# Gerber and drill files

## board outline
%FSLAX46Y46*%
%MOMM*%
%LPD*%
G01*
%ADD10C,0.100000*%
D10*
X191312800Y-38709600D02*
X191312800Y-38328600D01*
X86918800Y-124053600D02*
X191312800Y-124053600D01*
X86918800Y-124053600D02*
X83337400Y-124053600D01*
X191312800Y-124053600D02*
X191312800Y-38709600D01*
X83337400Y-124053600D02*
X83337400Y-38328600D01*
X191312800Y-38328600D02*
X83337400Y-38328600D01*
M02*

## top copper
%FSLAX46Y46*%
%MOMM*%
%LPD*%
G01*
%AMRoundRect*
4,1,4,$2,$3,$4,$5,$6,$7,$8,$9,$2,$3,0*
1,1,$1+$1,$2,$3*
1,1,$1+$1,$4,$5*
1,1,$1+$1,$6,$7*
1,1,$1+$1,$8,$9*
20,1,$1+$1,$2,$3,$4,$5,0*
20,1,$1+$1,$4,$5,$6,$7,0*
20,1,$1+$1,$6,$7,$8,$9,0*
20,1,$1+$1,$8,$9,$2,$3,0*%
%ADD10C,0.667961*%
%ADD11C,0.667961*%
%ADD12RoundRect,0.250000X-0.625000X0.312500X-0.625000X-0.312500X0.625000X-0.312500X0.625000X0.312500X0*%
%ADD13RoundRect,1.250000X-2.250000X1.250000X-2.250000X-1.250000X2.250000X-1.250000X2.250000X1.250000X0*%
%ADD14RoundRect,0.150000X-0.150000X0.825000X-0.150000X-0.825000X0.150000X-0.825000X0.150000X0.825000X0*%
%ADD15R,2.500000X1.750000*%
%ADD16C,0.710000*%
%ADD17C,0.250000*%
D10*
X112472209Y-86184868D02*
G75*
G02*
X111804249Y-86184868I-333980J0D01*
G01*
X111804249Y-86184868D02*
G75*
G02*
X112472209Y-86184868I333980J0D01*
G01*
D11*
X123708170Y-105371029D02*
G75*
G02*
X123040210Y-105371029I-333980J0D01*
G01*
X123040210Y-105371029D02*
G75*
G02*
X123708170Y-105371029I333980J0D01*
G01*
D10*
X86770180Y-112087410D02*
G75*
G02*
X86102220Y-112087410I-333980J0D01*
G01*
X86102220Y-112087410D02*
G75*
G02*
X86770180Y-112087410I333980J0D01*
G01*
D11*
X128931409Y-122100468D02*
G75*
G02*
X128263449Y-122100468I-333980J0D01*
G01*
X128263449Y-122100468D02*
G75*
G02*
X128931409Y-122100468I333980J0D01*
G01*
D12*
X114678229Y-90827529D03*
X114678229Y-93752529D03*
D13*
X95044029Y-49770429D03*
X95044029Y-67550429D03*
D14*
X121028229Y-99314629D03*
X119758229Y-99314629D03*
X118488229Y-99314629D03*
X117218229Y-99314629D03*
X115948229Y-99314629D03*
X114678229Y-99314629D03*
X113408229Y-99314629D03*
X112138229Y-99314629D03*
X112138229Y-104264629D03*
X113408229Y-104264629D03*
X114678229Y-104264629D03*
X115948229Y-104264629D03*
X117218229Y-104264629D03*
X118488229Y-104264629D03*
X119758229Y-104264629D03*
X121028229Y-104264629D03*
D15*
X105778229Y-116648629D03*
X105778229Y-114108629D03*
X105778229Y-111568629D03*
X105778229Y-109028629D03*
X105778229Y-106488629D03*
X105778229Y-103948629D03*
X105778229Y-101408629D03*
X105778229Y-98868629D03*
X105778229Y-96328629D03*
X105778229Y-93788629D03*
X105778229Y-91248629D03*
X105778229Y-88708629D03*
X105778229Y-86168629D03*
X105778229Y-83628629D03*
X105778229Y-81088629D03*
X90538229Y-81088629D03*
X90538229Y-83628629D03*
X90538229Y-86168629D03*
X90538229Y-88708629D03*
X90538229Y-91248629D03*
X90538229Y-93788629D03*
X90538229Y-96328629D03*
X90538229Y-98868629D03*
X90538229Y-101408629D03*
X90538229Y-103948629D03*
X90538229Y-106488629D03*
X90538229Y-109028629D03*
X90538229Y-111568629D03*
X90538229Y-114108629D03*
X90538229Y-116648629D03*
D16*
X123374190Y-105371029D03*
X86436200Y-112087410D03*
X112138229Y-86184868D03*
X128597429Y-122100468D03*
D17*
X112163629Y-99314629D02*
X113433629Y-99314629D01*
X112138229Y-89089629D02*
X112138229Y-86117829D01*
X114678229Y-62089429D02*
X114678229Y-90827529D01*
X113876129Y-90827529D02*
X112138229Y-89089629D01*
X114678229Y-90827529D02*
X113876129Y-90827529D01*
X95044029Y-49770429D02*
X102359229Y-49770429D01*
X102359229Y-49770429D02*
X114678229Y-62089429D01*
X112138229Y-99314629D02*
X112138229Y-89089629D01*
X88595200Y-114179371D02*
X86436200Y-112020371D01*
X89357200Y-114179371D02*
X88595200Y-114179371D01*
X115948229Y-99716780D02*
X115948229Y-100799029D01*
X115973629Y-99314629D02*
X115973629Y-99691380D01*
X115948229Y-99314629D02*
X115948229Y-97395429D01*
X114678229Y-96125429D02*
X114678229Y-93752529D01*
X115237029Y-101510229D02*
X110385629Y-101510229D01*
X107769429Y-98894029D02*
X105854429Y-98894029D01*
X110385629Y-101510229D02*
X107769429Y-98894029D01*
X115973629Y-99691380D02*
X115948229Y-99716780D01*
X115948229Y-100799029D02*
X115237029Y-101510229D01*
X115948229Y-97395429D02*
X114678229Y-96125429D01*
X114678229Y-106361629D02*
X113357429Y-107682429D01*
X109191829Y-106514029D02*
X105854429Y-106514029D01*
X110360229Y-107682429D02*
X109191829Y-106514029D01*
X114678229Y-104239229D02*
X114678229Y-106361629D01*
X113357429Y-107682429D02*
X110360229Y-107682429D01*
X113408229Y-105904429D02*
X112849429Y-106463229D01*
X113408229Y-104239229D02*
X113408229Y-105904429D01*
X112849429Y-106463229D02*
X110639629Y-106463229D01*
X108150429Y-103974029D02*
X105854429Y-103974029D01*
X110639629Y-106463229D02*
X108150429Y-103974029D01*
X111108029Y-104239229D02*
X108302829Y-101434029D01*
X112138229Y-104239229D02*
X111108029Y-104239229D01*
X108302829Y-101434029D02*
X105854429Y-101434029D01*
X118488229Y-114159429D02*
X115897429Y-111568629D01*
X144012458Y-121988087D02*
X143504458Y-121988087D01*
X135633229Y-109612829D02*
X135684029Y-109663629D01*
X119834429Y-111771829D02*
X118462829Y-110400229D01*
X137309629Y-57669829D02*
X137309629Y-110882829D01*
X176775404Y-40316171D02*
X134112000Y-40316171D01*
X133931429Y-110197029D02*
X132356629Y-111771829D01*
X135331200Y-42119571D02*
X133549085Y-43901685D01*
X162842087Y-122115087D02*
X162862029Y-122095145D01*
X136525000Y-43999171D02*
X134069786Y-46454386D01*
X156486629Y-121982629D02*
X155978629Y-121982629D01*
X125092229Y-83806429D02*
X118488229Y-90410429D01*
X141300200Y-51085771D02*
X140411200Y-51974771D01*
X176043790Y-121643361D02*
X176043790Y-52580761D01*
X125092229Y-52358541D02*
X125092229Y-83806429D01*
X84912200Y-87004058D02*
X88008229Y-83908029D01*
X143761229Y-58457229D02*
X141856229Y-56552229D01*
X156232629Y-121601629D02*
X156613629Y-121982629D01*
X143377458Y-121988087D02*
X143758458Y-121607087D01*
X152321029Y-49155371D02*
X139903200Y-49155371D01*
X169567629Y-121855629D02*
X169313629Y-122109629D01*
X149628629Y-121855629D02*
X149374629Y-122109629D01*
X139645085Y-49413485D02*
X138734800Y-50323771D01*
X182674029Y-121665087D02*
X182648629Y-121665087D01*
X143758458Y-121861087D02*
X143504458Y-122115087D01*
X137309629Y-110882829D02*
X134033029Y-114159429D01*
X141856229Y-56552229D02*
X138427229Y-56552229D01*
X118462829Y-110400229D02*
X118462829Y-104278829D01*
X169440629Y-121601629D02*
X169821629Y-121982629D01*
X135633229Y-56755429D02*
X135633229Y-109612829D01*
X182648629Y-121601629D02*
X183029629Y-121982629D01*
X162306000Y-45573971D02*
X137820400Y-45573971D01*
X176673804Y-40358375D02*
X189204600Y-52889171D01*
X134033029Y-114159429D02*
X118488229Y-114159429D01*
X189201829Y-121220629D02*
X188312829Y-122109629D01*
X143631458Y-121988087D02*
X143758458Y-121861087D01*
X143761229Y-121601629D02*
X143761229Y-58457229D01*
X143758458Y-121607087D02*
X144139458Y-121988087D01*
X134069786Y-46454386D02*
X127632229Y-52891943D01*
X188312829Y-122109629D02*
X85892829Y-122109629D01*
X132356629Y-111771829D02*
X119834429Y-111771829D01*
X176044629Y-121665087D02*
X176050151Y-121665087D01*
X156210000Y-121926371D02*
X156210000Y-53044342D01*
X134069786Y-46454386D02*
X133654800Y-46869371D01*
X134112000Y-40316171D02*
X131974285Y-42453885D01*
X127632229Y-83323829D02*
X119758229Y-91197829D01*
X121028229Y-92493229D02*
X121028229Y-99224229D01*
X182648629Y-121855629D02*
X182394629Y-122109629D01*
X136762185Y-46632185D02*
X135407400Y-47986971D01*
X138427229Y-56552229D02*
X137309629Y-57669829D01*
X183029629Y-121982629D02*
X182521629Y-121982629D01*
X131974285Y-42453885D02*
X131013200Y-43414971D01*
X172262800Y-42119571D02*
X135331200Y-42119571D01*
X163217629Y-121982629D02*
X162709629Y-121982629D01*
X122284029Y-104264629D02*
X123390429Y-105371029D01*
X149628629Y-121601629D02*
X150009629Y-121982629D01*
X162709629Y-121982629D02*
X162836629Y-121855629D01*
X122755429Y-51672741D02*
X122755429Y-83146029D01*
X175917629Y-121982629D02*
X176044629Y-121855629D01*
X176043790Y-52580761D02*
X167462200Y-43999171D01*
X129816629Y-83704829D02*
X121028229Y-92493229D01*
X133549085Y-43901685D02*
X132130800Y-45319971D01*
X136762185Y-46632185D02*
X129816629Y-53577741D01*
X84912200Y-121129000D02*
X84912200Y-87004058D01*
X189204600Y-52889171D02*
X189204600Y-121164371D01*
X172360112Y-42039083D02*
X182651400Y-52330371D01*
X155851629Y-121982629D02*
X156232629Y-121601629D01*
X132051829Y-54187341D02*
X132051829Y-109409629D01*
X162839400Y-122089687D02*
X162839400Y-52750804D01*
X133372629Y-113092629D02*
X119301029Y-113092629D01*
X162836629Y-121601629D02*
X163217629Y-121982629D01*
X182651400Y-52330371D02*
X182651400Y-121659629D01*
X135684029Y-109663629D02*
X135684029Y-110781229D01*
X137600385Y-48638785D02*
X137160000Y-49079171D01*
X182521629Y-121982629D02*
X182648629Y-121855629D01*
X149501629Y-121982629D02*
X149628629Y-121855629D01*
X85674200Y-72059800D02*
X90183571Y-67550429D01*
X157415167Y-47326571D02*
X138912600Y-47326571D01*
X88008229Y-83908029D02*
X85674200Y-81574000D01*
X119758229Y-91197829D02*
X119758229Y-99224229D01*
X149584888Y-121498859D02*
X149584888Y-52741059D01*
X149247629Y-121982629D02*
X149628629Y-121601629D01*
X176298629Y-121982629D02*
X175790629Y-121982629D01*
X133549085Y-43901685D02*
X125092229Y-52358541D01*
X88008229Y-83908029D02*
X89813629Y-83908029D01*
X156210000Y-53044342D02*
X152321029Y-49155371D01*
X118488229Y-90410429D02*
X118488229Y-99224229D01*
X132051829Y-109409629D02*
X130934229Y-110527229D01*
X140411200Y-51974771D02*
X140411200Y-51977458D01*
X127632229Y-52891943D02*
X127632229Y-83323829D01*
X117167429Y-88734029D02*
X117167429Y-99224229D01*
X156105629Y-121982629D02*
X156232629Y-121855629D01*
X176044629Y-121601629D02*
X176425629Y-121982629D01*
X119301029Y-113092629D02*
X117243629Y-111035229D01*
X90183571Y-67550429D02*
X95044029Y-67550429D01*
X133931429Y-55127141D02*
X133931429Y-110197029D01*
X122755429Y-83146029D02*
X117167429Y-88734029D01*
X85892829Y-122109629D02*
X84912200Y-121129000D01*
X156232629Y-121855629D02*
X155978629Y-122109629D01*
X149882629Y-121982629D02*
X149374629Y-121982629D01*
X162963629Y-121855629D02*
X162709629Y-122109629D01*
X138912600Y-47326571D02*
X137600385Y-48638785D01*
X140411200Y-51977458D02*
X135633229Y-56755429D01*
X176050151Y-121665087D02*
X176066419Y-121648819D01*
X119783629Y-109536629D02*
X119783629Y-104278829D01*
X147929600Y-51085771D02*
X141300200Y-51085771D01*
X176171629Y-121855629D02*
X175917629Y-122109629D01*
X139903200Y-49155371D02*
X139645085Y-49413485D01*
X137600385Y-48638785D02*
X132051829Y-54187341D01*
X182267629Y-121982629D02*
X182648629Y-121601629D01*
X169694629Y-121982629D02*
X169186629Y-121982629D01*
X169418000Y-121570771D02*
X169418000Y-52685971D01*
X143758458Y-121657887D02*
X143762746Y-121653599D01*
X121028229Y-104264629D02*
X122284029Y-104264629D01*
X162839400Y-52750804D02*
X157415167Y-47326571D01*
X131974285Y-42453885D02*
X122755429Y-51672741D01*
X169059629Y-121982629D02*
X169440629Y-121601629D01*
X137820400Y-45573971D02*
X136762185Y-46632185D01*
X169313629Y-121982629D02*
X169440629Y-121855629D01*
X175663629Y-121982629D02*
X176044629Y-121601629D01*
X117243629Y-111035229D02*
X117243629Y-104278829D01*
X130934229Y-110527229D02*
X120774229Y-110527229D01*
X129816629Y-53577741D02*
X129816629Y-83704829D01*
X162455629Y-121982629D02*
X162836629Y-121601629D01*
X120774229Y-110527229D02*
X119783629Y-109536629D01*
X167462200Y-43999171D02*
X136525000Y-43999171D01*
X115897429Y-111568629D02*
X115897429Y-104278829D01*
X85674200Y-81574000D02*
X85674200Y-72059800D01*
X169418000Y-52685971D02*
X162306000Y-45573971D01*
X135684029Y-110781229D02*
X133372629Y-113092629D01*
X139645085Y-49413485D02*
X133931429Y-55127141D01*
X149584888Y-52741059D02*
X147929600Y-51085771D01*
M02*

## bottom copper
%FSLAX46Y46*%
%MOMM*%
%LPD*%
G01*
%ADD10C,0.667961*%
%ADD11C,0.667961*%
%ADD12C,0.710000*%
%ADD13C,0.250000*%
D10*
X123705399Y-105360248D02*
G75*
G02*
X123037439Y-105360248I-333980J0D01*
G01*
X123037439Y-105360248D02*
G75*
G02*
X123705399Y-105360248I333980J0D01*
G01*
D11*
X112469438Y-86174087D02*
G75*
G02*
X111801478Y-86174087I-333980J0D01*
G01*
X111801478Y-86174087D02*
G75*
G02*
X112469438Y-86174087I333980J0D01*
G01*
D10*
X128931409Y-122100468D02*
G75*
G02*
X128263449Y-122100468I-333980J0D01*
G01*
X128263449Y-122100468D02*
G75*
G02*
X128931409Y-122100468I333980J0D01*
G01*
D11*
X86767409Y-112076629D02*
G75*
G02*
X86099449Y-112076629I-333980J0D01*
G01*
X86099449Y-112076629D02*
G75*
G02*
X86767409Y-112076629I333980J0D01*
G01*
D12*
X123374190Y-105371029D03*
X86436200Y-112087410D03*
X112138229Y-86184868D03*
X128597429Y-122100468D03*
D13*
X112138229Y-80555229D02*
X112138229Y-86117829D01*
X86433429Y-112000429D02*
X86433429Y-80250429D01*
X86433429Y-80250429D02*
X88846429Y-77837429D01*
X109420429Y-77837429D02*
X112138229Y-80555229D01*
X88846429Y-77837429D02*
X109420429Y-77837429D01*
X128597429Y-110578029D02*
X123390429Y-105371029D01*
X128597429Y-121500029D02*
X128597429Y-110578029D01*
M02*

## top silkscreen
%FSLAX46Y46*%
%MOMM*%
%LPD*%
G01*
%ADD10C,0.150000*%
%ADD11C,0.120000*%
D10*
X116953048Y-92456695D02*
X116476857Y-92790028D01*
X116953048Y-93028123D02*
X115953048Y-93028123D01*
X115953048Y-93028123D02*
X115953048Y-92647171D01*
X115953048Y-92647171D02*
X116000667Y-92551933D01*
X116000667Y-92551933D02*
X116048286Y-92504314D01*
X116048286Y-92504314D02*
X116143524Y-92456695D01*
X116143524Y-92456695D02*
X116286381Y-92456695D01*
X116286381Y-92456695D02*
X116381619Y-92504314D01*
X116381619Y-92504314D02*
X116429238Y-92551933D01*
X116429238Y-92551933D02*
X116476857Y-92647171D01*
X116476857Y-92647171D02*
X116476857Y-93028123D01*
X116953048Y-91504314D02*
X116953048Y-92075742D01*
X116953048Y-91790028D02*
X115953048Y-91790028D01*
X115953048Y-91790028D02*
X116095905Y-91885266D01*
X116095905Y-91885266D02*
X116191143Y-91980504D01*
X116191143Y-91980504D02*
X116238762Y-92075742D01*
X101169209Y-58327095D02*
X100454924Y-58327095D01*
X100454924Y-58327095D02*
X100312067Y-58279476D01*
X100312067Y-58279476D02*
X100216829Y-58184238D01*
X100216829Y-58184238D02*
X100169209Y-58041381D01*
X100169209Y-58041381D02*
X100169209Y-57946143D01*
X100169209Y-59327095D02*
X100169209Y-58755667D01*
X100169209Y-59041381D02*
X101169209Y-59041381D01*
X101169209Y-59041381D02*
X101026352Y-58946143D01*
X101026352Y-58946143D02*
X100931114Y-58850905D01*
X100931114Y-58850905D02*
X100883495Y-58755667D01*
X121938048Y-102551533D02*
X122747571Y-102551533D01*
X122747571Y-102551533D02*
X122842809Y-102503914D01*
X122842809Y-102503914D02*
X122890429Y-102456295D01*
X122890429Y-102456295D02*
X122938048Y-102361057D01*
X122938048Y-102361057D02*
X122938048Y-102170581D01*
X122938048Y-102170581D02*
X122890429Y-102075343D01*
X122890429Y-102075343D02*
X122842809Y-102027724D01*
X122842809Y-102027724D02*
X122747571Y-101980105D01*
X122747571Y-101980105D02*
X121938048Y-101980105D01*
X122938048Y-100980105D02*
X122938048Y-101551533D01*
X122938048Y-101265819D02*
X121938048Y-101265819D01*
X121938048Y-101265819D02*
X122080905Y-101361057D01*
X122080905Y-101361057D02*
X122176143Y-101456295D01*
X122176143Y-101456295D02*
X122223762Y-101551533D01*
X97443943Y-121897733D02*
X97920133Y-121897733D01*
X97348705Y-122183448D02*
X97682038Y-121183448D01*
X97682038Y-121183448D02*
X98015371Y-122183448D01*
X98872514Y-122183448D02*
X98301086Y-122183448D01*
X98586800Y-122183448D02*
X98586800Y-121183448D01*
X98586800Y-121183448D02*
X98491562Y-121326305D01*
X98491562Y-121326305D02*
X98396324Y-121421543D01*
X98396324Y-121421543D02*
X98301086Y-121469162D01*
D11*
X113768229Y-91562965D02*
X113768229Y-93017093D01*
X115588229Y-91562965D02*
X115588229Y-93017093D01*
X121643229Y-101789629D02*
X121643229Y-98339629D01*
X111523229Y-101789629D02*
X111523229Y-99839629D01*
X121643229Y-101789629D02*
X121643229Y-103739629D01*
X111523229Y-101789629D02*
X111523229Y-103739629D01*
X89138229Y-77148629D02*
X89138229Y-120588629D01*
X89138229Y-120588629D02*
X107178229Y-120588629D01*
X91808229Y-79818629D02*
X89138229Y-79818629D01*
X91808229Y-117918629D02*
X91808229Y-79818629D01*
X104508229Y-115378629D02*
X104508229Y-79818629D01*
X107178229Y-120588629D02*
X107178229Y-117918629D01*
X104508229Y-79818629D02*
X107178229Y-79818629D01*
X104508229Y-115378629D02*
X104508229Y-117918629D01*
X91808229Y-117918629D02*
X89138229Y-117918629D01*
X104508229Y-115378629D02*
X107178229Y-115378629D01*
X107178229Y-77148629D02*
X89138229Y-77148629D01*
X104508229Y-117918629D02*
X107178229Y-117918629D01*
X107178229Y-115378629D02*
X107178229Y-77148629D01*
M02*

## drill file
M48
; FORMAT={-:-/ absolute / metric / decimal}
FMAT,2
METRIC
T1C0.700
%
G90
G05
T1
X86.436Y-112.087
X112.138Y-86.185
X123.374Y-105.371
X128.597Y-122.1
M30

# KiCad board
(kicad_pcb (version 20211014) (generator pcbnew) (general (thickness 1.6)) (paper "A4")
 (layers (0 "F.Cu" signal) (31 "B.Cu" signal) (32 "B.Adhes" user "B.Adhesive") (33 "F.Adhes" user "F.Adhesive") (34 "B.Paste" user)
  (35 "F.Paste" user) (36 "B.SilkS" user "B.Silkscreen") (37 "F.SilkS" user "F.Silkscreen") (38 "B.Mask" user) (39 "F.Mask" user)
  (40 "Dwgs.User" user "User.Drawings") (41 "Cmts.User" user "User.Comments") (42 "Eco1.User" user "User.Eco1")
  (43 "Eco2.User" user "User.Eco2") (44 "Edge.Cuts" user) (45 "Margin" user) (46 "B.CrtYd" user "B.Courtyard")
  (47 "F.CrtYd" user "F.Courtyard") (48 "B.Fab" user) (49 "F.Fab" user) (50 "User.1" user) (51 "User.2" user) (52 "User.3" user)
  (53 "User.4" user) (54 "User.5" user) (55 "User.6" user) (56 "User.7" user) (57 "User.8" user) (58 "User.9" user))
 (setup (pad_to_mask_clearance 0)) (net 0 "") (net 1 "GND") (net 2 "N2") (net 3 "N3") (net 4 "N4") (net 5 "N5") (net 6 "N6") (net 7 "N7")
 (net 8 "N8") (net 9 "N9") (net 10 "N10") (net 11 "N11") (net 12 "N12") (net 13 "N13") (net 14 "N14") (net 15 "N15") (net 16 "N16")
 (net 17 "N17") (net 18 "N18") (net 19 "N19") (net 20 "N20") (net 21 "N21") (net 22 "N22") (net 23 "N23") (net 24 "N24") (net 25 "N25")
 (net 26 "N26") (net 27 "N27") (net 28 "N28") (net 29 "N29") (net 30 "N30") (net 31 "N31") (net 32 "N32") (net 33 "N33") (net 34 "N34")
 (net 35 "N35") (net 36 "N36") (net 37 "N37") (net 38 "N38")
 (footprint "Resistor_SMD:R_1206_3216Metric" (layer "F.Cu") (at 114.678229 92.290029 -90)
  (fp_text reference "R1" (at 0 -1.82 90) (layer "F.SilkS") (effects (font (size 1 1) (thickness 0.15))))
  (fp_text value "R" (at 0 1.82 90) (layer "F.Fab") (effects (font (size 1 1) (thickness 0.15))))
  (fp_line (start -0.727064 0.91) (end 0.727064 0.91) (layer "F.SilkS") (width 0.12))
  (fp_line (start -0.727064 -0.91) (end 0.727064 -0.91) (layer "F.SilkS") (width 0.12))
  (pad "1" smd roundrect (at -1.4625 0 270) (size 1.125 1.75) (layers "F.Cu" "F.Paste" "F.Mask") (roundrect_rratio 0.222222) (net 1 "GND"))
  (pad "2" smd roundrect (at 1.4625 0 270) (size 1.125 1.75) (layers "F.Cu" "F.Paste" "F.Mask") (roundrect_rratio 0.222222) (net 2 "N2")))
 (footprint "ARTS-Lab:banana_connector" (layer "F.Cu") (at 100.124029 58.660429 -90)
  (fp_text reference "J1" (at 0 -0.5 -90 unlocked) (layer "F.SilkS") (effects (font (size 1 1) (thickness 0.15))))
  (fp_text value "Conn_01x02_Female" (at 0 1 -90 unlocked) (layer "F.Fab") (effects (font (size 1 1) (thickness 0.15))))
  (pad "1" smd roundrect (at -8.89 5.08 270) (size 5 7) (layers "F.Cu" "F.Paste" "F.Mask") (roundrect_rratio 0.25) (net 1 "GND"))
  (pad "2" smd roundrect (at 8.89 5.08 270) (size 5 7) (layers "F.Cu" "F.Paste" "F.Mask") (roundrect_rratio 0.25) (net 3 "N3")))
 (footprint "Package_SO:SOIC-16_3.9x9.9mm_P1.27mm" (layer "F.Cu") (at 116.583229 101.789629 -90)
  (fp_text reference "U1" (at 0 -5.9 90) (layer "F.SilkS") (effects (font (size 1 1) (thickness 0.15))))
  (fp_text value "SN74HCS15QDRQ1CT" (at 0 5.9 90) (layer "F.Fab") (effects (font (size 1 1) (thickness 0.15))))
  (fp_line (start 0 -5.06) (end -3.45 -5.06) (layer "F.SilkS") (width 0.12))
  (fp_line (start 0 5.06) (end -1.95 5.06) (layer "F.SilkS") (width 0.12))
  (fp_line (start 0 -5.06) (end 1.95 -5.06) (layer "F.SilkS") (width 0.12))
  (fp_line (start 0 5.06) (end 1.95 5.06) (layer "F.SilkS") (width 0.12))
  (pad "1" smd roundrect (at -2.475 -4.445 270) (size 1.95 0.6) (layers "F.Cu" "F.Paste" "F.Mask") (roundrect_rratio 0.25) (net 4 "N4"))
  (pad "2" smd roundrect (at -2.475 -3.175 270) (size 1.95 0.6) (layers "F.Cu" "F.Paste" "F.Mask") (roundrect_rratio 0.25) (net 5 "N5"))
  (pad "3" smd roundrect (at -2.475 -1.905 270) (size 1.95 0.6) (layers "F.Cu" "F.Paste" "F.Mask") (roundrect_rratio 0.25) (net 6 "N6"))
  (pad "4" smd roundrect (at -2.475 -0.635 270) (size 1.95 0.6) (layers "F.Cu" "F.Paste" "F.Mask") (roundrect_rratio 0.25) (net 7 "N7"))
  (pad "5" smd roundrect (at -2.475 0.635 270) (size 1.95 0.6) (layers "F.Cu" "F.Paste" "F.Mask") (roundrect_rratio 0.25) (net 2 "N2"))
  (pad "6" smd roundrect (at -2.475 1.905 270) (size 1.95 0.6) (layers "F.Cu" "F.Paste" "F.Mask") (roundrect_rratio 0.25) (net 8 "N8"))
  (pad "7" smd roundrect (at -2.475 3.175 270) (size 1.95 0.6) (layers "F.Cu" "F.Paste" "F.Mask") (roundrect_rratio 0.25) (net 1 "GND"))
  (pad "8" smd roundrect (at -2.475 4.445 270) (size 1.95 0.6) (layers "F.Cu" "F.Paste" "F.Mask") (roundrect_rratio 0.25) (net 1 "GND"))
  (pad "9" smd roundrect (at 2.475 4.445 270) (size 1.95 0.6) (layers "F.Cu" "F.Paste" "F.Mask") (roundrect_rratio 0.25) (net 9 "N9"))
  (pad "10" smd roundrect (at 2.475 3.175 270) (size 1.95 0.6) (layers "F.Cu" "F.Paste" "F.Mask") (roundrect_rratio 0.25) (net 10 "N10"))
  (pad "11" smd roundrect (at 2.475 1.905 270) (size 1.95 0.6) (layers "F.Cu" "F.Paste" "F.Mask") (roundrect_rratio 0.25) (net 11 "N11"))
  (pad "12" smd roundrect (at 2.475 0.635 270) (size 1.95 0.6) (layers "F.Cu" "F.Paste" "F.Mask") (roundrect_rratio 0.25) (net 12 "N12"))
  (pad "13" smd roundrect (at 2.475 -0.635 270) (size 1.95 0.6) (layers "F.Cu" "F.Paste" "F.Mask") (roundrect_rratio 0.25) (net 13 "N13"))
  (pad "14" smd roundrect (at 2.475 -1.905 270) (size 1.95 0.6) (layers "F.Cu" "F.Paste" "F.Mask") (roundrect_rratio 0.25) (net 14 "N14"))
  (pad "15" smd roundrect (at 2.475 -3.175 270) (size 1.95 0.6) (layers "F.Cu" "F.Paste" "F.Mask") (roundrect_rratio 0.25) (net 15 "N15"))
  (pad "16" smd roundrect (at 2.475 -4.445 270) (size 1.95 0.6) (layers "F.Cu" "F.Paste" "F.Mask") (roundrect_rratio 0.25) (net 3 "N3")))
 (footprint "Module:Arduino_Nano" (layer "F.Cu") (at 105.778229 116.648629 180)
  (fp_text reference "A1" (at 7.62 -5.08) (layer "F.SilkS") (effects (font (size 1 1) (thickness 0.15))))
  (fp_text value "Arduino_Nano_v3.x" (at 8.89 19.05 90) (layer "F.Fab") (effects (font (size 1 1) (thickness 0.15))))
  (fp_line (start 16.64 39.5) (end 16.64 -3.94) (layer "F.SilkS") (width 0.12))
  (fp_line (start 16.64 -3.94) (end -1.4 -3.94) (layer "F.SilkS") (width 0.12))
  (fp_line (start 13.97 36.83) (end 16.64 36.83) (layer "F.SilkS") (width 0.12))
  (fp_line (start 13.97 -1.27) (end 13.97 36.83) (layer "F.SilkS") (width 0.12))
  (fp_line (start 1.27 1.27) (end 1.27 36.83) (layer "F.SilkS") (width 0.12))
  (fp_line (start -1.4 -3.94) (end -1.4 -1.27) (layer "F.SilkS") (width 0.12))
  (fp_line (start 1.27 36.83) (end -1.4 36.83) (layer "F.SilkS") (width 0.12))
  (fp_line (start 1.27 1.27) (end 1.27 -1.27) (layer "F.SilkS") (width 0.12))
  (fp_line (start 13.97 -1.27) (end 16.64 -1.27) (layer "F.SilkS") (width 0.12))
  (fp_line (start 1.27 1.27) (end -1.4 1.27) (layer "F.SilkS") (width 0.12))
  (fp_line (start -1.4 39.5) (end 16.64 39.5) (layer "F.SilkS") (width 0.12))
  (fp_line (start 1.27 -1.27) (end -1.4 -1.27) (layer "F.SilkS") (width 0.12))
  (fp_line (start -1.4 1.27) (end -1.4 39.5) (layer "F.SilkS") (width 0.12))
  (pad "1" smd rect (at 0 0 180) (size 2.5 1.75) (layers "F.Cu" "F.Paste" "F.Mask") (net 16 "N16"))
  (pad "2" smd rect (at 0 2.54 180) (size 2.5 1.75) (layers "F.Cu" "F.Paste" "F.Mask") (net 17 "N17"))
  (pad "3" smd rect (at 0 5.08 180) (size 2.5 1.75) (layers "F.Cu" "F.Paste" "F.Mask") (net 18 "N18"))
  (pad "4" smd rect (at 0 7.62 180) (size 2.5 1.75) (layers "F.Cu" "F.Paste" "F.Mask") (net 1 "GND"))
  (pad "5" smd rect (at 0 10.16 180) (size 2.5 1.75) (layers "F.Cu" "F.Paste" "F.Mask") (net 11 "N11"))
  (pad "6" smd rect (at 0 12.7 180) (size 2.5 1.75) (layers "F.Cu" "F.Paste" "F.Mask") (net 10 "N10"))
  (pad "7" smd rect (at 0 15.24 180) (size 2.5 1.75) (layers "F.Cu" "F.Paste" "F.Mask") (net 9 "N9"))
  (pad "8" smd rect (at 0 17.78 180) (size 2.5 1.75) (layers "F.Cu" "F.Paste" "F.Mask") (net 2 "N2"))
  (pad "9" smd rect (at 0 20.32 180) (size 2.5 1.75) (layers "F.Cu" "F.Paste" "F.Mask") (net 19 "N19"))
  (pad "10" smd rect (at 0 22.86 180) (size 2.5 1.75) (layers "F.Cu" "F.Paste" "F.Mask") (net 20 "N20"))
  (pad "11" smd rect (at 0 25.4 180) (size 2.5 1.75) (layers "F.Cu" "F.Paste" "F.Mask") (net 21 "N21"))
  (pad "12" smd rect (at 0 27.94 180) (size 2.5 1.75) (layers "F.Cu" "F.Paste" "F.Mask") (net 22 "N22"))
  (pad "13" smd rect (at 0 30.48 180) (size 2.5 1.75) (layers "F.Cu" "F.Paste" "F.Mask") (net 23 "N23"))
  (pad "14" smd rect (at 0 33.02 180) (size 2.5 1.75) (layers "F.Cu" "F.Paste" "F.Mask") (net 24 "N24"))
  (pad "15" smd rect (at 0 35.56 180) (size 2.5 1.75) (layers "F.Cu" "F.Paste" "F.Mask") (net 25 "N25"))
  (pad "16" smd rect (at 15.24 35.56 180) (size 2.5 1.75) (layers "F.Cu" "F.Paste" "F.Mask") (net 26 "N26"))
  (pad "17" smd rect (at 15.24 33.02 180) (size 2.5 1.75) (layers "F.Cu" "F.Paste" "F.Mask") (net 3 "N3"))
  (pad "18" smd rect (at 15.24 30.48 180) (size 2.5 1.75) (layers "F.Cu" "F.Paste" "F.Mask") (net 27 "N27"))
  (pad "19" smd rect (at 15.24 27.94 180) (size 2.5 1.75) (layers "F.Cu" "F.Paste" "F.Mask") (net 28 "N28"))
  (pad "20" smd rect (at 15.24 25.4 180) (size 2.5 1.75) (layers "F.Cu" "F.Paste" "F.Mask") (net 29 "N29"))
  (pad "21" smd rect (at 15.24 22.86 180) (size 2.5 1.75) (layers "F.Cu" "F.Paste" "F.Mask") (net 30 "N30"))
  (pad "22" smd rect (at 15.24 20.32 180) (size 2.5 1.75) (layers "F.Cu" "F.Paste" "F.Mask") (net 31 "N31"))
  (pad "23" smd rect (at 15.24 17.78 180) (size 2.5 1.75) (layers "F.Cu" "F.Paste" "F.Mask") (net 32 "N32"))
  (pad "24" smd rect (at 15.24 15.24 180) (size 2.5 1.75) (layers "F.Cu" "F.Paste" "F.Mask") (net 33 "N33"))
  (pad "25" smd rect (at 15.24 12.7 180) (size 2.5 1.75) (layers "F.Cu" "F.Paste" "F.Mask") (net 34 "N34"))
  (pad "26" smd rect (at 15.24 10.16 180) (size 2.5 1.75) (layers "F.Cu" "F.Paste" "F.Mask") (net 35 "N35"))
  (pad "27" smd rect (at 15.24 7.62 180) (size 2.5 1.75) (layers "F.Cu" "F.Paste" "F.Mask") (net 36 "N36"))
  (pad "28" smd rect (at 15.24 5.08 180) (size 2.5 1.75) (layers "F.Cu" "F.Paste" "F.Mask") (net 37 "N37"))
  (pad "29" smd rect (at 15.24 2.54 180) (size 2.5 1.75) (layers "F.Cu" "F.Paste" "F.Mask") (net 1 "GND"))
  (pad "30" smd rect (at 15.24 0 180) (size 2.5 1.75) (layers "F.Cu" "F.Paste" "F.Mask") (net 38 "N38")))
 (gr_circle (center 112.138229 86.184868) (end 112.70619 86.184868) (layer "F.Cu") (width 0.2) (fill solid))
 (gr_circle (center 123.37419 105.371029) (end 123.942151 105.371029) (layer "F.Cu") (width 0.2) (fill solid))
 (gr_circle (center 86.4362 112.08741) (end 87.004161 112.08741) (layer "F.Cu") (width 0.2) (fill solid))
 (gr_circle (center 128.597429 122.100468) (end 129.16539 122.100468) (layer "F.Cu") (width 0.2) (fill solid))
 (gr_circle (center 123.371419 105.360248) (end 123.93938 105.360248) (layer "B.Cu") (width 0.2) (fill solid))
 (gr_circle (center 112.135458 86.174087) (end 112.703419 86.174087) (layer "B.Cu") (width 0.2) (fill solid))
 (gr_circle (center 128.597429 122.100468) (end 129.16539 122.100468) (layer "B.Cu") (width 0.2) (fill solid))
 (gr_circle (center 86.433429 112.076629) (end 87.00139 112.076629) (layer "B.Cu") (width 0.2) (fill solid))
 (gr_line (start 191.3128 38.7096) (end 191.3128 38.3286) (layer "Edge.Cuts") (width 0.1))
 (gr_line (start 86.9188 124.0536) (end 191.3128 124.0536) (layer "Edge.Cuts") (width 0.1))
 (gr_line (start 86.9188 124.0536) (end 83.3374 124.0536) (layer "Edge.Cuts") (width 0.1))
 (gr_line (start 191.3128 124.0536) (end 191.3128 38.7096) (layer "Edge.Cuts") (width 0.1))
 (gr_line (start 83.3374 124.0536) (end 83.3374 38.3286) (layer "Edge.Cuts") (width 0.1))
 (gr_line (start 191.3128 38.3286) (end 83.3374 38.3286) (layer "Edge.Cuts") (width 0.1))
 (via (at 123.37419 105.371029) (size 0.71) (drill 0.7) (layers "F.Cu" "B.Cu") (free) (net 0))
 (via (at 86.4362 112.08741) (size 0.71) (drill 0.7) (layers "F.Cu" "B.Cu") (free) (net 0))
 (via (at 112.138229 86.184868) (size 0.71) (drill 0.7) (layers "F.Cu" "B.Cu") (free) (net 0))
 (via (at 128.597429 122.100468) (size 0.71) (drill 0.7) (layers "F.Cu" "B.Cu") (free) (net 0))
 (segment (start 112.163629 99.314629) (end 113.433629 99.314629) (width 0.25) (layer "F.Cu") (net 1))
 (segment (start 112.138229 89.089629) (end 112.138229 86.117829) (width 0.25) (layer "F.Cu") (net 1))
 (segment (start 114.678229 62.089429) (end 114.678229 90.827529) (width 0.25) (layer "F.Cu") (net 1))
 (segment (start 113.876129 90.827529) (end 112.138229 89.089629) (width 0.25) (layer "F.Cu") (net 1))
 (segment (start 114.678229 90.827529) (end 113.876129 90.827529) (width 0.25) (layer "F.Cu") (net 1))
 (segment (start 95.044029 49.770429) (end 102.359229 49.770429) (width 0.25) (layer "F.Cu") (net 1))
 (segment (start 102.359229 49.770429) (end 114.678229 62.089429) (width 0.25) (layer "F.Cu") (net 1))
 (segment (start 112.138229 99.314629) (end 112.138229 89.089629) (width 0.25) (layer "F.Cu") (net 1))
 (segment (start 88.5952 114.179371) (end 86.4362 112.020371) (width 0.25) (layer "F.Cu") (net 1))
 (segment (start 89.3572 114.179371) (end 88.5952 114.179371) (width 0.25) (layer "F.Cu") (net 1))
 (segment (start 112.138229 80.555229) (end 112.138229 86.117829) (width 0.25) (layer "B.Cu") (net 1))
 (segment (start 86.433429 112.000429) (end 86.433429 80.250429) (width 0.25) (layer "B.Cu") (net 1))
 (segment (start 86.433429 80.250429) (end 88.846429 77.837429) (width 0.25) (layer "B.Cu") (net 1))
 (segment (start 109.420429 77.837429) (end 112.138229 80.555229) (width 0.25) (layer "B.Cu") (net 1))
 (segment (start 88.846429 77.837429) (end 109.420429 77.837429) (width 0.25) (layer "B.Cu") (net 1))
 (segment (start 115.948229 99.71678) (end 115.948229 100.799029) (width 0.25) (layer "F.Cu") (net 2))
 (segment (start 115.973629 99.314629) (end 115.973629 99.69138) (width 0.25) (layer "F.Cu") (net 2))
 (segment (start 115.948229 99.314629) (end 115.948229 97.395429) (width 0.25) (layer "F.Cu") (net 2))
 (segment (start 114.678229 96.125429) (end 114.678229 93.752529) (width 0.25) (layer "F.Cu") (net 2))
 (segment (start 115.237029 101.510229) (end 110.385629 101.510229) (width 0.25) (layer "F.Cu") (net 2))
 (segment (start 107.769429 98.894029) (end 105.854429 98.894029) (width 0.25) (layer "F.Cu") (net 2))
 (segment (start 110.385629 101.510229) (end 107.769429 98.894029) (width 0.25) (layer "F.Cu") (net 2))
 (segment (start 115.973629 99.69138) (end 115.948229 99.71678) (width 0.25) (layer "F.Cu") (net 2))
 (segment (start 115.948229 100.799029) (end 115.237029 101.510229) (width 0.25) (layer "F.Cu") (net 2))
 (segment (start 115.948229 97.395429) (end 114.678229 96.125429) (width 0.25) (layer "F.Cu") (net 2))
 (segment (start 114.678229 106.361629) (end 113.357429 107.682429) (width 0.25) (layer "F.Cu") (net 11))
 (segment (start 109.191829 106.514029) (end 105.854429 106.514029) (width 0.25) (layer "F.Cu") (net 11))
 (segment (start 110.360229 107.682429) (end 109.191829 106.514029) (width 0.25) (layer "F.Cu") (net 11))
 (segment (start 114.678229 104.239229) (end 114.678229 106.361629) (width 0.25) (layer "F.Cu") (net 11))
 (segment (start 113.357429 107.682429) (end 110.360229 107.682429) (width 0.25) (layer "F.Cu") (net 11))
 (segment (start 113.408229 105.904429) (end 112.849429 106.463229) (width 0.25) (layer "F.Cu") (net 10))
 (segment (start 113.408229 104.239229) (end 113.408229 105.904429) (width 0.25) (layer "F.Cu") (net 10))
 (segment (start 112.849429 106.463229) (end 110.639629 106.463229) (width 0.25) (layer "F.Cu") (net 10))
 (segment (start 108.150429 103.974029) (end 105.854429 103.974029) (width 0.25) (layer "F.Cu") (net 10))
 (segment (start 110.639629 106.463229) (end 108.150429 103.974029) (width 0.25) (layer "F.Cu") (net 10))
 (segment (start 111.108029 104.239229) (end 108.302829 101.434029) (width 0.25) (layer "F.Cu") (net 9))
 (segment (start 112.138229 104.239229) (end 111.108029 104.239229) (width 0.25) (layer "F.Cu") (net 9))
 (segment (start 108.302829 101.434029) (end 105.854429 101.434029) (width 0.25) (layer "F.Cu") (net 9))
 (segment (start 118.488229 114.159429) (end 115.897429 111.568629) (width 0.25) (layer "F.Cu") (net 3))
 (segment (start 144.012458 121.988087) (end 143.504458 121.988087) (width 0.25) (layer "F.Cu") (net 3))
 (segment (start 135.633229 109.612829) (end 135.684029 109.663629) (width 0.25) (layer "F.Cu") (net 3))
 (segment (start 119.834429 111.771829) (end 118.462829 110.400229) (width 0.25) (layer "F.Cu") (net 3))
 (segment (start 137.309629 57.669829) (end 137.309629 110.882829) (width 0.25) (layer "F.Cu") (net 3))
 (segment (start 176.775404 40.316171) (end 134.112 40.316171) (width 0.25) (layer "F.Cu") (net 3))
 (segment (start 133.931429 110.197029) (end 132.356629 111.771829) (width 0.25) (layer "F.Cu") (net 3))
 (segment (start 135.3312 42.119571) (end 133.549085 43.901685) (width 0.25) (layer "F.Cu") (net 3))
 (segment (start 162.842087 122.115087) (end 162.862029 122.095145) (width 0.25) (layer "F.Cu") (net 3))
 (segment (start 136.525 43.999171) (end 134.069786 46.454386) (width 0.25) (layer "F.Cu") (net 3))
 (segment (start 156.486629 121.982629) (end 155.978629 121.982629) (width 0.25) (layer "F.Cu") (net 3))
 (segment (start 125.092229 83.806429) (end 118.488229 90.410429) (width 0.25) (layer "F.Cu") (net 3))
 (segment (start 141.3002 51.085771) (end 140.4112 51.974771) (width 0.25) (layer "F.Cu") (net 3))
 (segment (start 176.04379 121.643361) (end 176.04379 52.580761) (width 0.25) (layer "F.Cu") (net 3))
 (segment (start 125.092229 52.358541) (end 125.092229 83.806429) (width 0.25) (layer "F.Cu") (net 3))
 (segment (start 84.9122 87.004058) (end 88.008229 83.908029) (width 0.25) (layer "F.Cu") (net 3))
 (segment (start 143.761229 58.457229) (end 141.856229 56.552229) (width 0.25) (layer "F.Cu") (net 3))
 (segment (start 156.232629 121.601629) (end 156.613629 121.982629) (width 0.25) (layer "F.Cu") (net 3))
 (segment (start 143.377458 121.988087) (end 143.758458 121.607087) (width 0.25) (layer "F.Cu") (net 3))
 (segment (start 152.321029 49.155371) (end 139.9032 49.155371) (width 0.25) (layer "F.Cu") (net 3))
 (segment (start 169.567629 121.855629) (end 169.313629 122.109629) (width 0.25) (layer "F.Cu") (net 3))
 (segment (start 149.628629 121.855629) (end 149.374629 122.109629) (width 0.25) (layer "F.Cu") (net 3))
 (segment (start 139.645085 49.413485) (end 138.7348 50.323771) (width 0.25) (layer "F.Cu") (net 3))
 (segment (start 182.674029 121.665087) (end 182.648629 121.665087) (width 0.25) (layer "F.Cu") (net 3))
 (segment (start 143.758458 121.861087) (end 143.504458 122.115087) (width 0.25) (layer "F.Cu") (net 3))
 (segment (start 137.309629 110.882829) (end 134.033029 114.159429) (width 0.25) (layer "F.Cu") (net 3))
 (segment (start 141.856229 56.552229) (end 138.427229 56.552229) (width 0.25) (layer "F.Cu") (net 3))
 (segment (start 118.462829 110.400229) (end 118.462829 104.278829) (width 0.25) (layer "F.Cu") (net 3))
 (segment (start 169.440629 121.601629) (end 169.821629 121.982629) (width 0.25) (layer "F.Cu") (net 3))
 (segment (start 135.633229 56.755429) (end 135.633229 109.612829) (width 0.25) (layer "F.Cu") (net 3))
 (segment (start 182.648629 121.601629) (end 183.029629 121.982629) (width 0.25) (layer "F.Cu") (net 3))
 (segment (start 162.306 45.573971) (end 137.8204 45.573971) (width 0.25) (layer "F.Cu") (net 3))
 (segment (start 176.673804 40.358375) (end 189.2046 52.889171) (width 0.25) (layer "F.Cu") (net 3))
 (segment (start 134.033029 114.159429) (end 118.488229 114.159429) (width 0.25) (layer "F.Cu") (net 3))
 (segment (start 189.201829 121.220629) (end 188.312829 122.109629) (width 0.25) (layer "F.Cu") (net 3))
 (segment (start 143.631458 121.988087) (end 143.758458 121.861087) (width 0.25) (layer "F.Cu") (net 3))
 (segment (start 143.761229 121.601629) (end 143.761229 58.457229) (width 0.25) (layer "F.Cu") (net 3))
 (segment (start 143.758458 121.607087) (end 144.139458 121.988087) (width 0.25) (layer "F.Cu") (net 3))
 (segment (start 134.069786 46.454386) (end 127.632229 52.891943) (width 0.25) (layer "F.Cu") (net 3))
 (segment (start 188.312829 122.109629) (end 85.892829 122.109629) (width 0.25) (layer "F.Cu") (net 3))
 (segment (start 132.356629 111.771829) (end 119.834429 111.771829) (width 0.25) (layer "F.Cu") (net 3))
 (segment (start 176.044629 121.665087) (end 176.050151 121.665087) (width 0.25) (layer "F.Cu") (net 3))
 (segment (start 156.21 121.926371) (end 156.21 53.044342) (width 0.25) (layer "F.Cu") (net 3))
 (segment (start 134.069786 46.454386) (end 133.6548 46.869371) (width 0.25) (layer "F.Cu") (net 3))
 (segment (start 134.112 40.316171) (end 131.974285 42.453885) (width 0.25) (layer "F.Cu") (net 3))
 (segment (start 127.632229 83.323829) (end 119.758229 91.197829) (width 0.25) (layer "F.Cu") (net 3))
 (segment (start 121.028229 92.493229) (end 121.028229 99.224229) (width 0.25) (layer "F.Cu") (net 3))
 (segment (start 182.648629 121.855629) (end 182.394629 122.109629) (width 0.25) (layer "F.Cu") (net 3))
 (segment (start 136.762185 46.632185) (end 135.4074 47.986971) (width 0.25) (layer "F.Cu") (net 3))
 (segment (start 138.427229 56.552229) (end 137.309629 57.669829) (width 0.25) (layer "F.Cu") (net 3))
 (segment (start 183.029629 121.982629) (end 182.521629 121.982629) (width 0.25) (layer "F.Cu") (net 3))
 (segment (start 131.974285 42.453885) (end 131.0132 43.414971) (width 0.25) (layer "F.Cu") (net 3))
 (segment (start 172.2628 42.119571) (end 135.3312 42.119571) (width 0.25) (layer "F.Cu") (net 3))
 (segment (start 163.217629 121.982629) (end 162.709629 121.982629) (width 0.25) (layer "F.Cu") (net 3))
 (segment (start 122.284029 104.264629) (end 123.390429 105.371029) (width 0.25) (layer "F.Cu") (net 3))
 (segment (start 149.628629 121.601629) (end 150.009629 121.982629) (width 0.25) (layer "F.Cu") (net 3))
 (segment (start 162.709629 121.982629) (end 162.836629 121.855629) (width 0.25) (layer "F.Cu") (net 3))
 (segment (start 122.755429 51.672741) (end 122.755429 83.146029) (width 0.25) (layer "F.Cu") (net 3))
 (segment (start 175.917629 121.982629) (end 176.044629 121.855629) (width 0.25) (layer "F.Cu") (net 3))
 (segment (start 176.04379 52.580761) (end 167.4622 43.999171) (width 0.25) (layer "F.Cu") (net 3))
 (segment (start 129.816629 83.704829) (end 121.028229 92.493229) (width 0.25) (layer "F.Cu") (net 3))
 (segment (start 133.549085 43.901685) (end 132.1308 45.319971) (width 0.25) (layer "F.Cu") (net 3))
 (segment (start 136.762185 46.632185) (end 129.816629 53.577741) (width 0.25) (layer "F.Cu") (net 3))
 (segment (start 84.9122 121.129) (end 84.9122 87.004058) (width 0.25) (layer "F.Cu") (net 3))
 (segment (start 189.2046 52.889171) (end 189.2046 121.164371) (width 0.25) (layer "F.Cu") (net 3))
 (segment (start 172.360112 42.039083) (end 182.6514 52.330371) (width 0.25) (layer "F.Cu") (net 3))
 (segment (start 155.851629 121.982629) (end 156.232629 121.601629) (width 0.25) (layer "F.Cu") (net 3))
 (segment (start 132.051829 54.187341) (end 132.051829 109.409629) (width 0.25) (layer "F.Cu") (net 3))
 (segment (start 162.8394 122.089687) (end 162.8394 52.750804) (width 0.25) (layer "F.Cu") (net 3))
 (segment (start 133.372629 113.092629) (end 119.301029 113.092629) (width 0.25) (layer "F.Cu") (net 3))
 (segment (start 162.836629 121.601629) (end 163.217629 121.982629) (width 0.25) (layer "F.Cu") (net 3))
 (segment (start 182.6514 52.330371) (end 182.6514 121.659629) (width 0.25) (layer "F.Cu") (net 3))
 (segment (start 135.684029 109.663629) (end 135.684029 110.781229) (width 0.25) (layer "F.Cu") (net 3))
 (segment (start 137.600385 48.638785) (end 137.16 49.079171) (width 0.25) (layer "F.Cu") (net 3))
 (segment (start 182.521629 121.982629) (end 182.648629 121.855629) (width 0.25) (layer "F.Cu") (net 3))
 (segment (start 149.501629 121.982629) (end 149.628629 121.855629) (width 0.25) (layer "F.Cu") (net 3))
 (segment (start 85.6742 72.0598) (end 90.183571 67.550429) (width 0.25) (layer "F.Cu") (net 3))
 (segment (start 157.415167 47.326571) (end 138.9126 47.326571) (width 0.25) (layer "F.Cu") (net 3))
 (segment (start 88.008229 83.908029) (end 85.6742 81.574) (width 0.25) (layer "F.Cu") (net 3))
 (segment (start 119.758229 91.197829) (end 119.758229 99.224229) (width 0.25) (layer "F.Cu") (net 3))
 (segment (start 149.584888 121.498859) (end 149.584888 52.741059) (width 0.25) (layer "F.Cu") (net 3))
 (segment (start 149.247629 121.982629) (end 149.628629 121.601629) (width 0.25) (layer "F.Cu") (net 3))
 (segment (start 176.298629 121.982629) (end 175.790629 121.982629) (width 0.25) (layer "F.Cu") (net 3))
 (segment (start 133.549085 43.901685) (end 125.092229 52.358541) (width 0.25) (layer "F.Cu") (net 3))
 (segment (start 88.008229 83.908029) (end 89.813629 83.908029) (width 0.25) (layer "F.Cu") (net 3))
 (segment (start 156.21 53.044342) (end 152.321029 49.155371) (width 0.25) (layer "F.Cu") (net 3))
 (segment (start 118.488229 90.410429) (end 118.488229 99.224229) (width 0.25) (layer "F.Cu") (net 3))
 (segment (start 132.051829 109.409629) (end 130.934229 110.527229) (width 0.25) (layer "F.Cu") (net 3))
 (segment (start 140.4112 51.974771) (end 140.4112 51.977458) (width 0.25) (layer "F.Cu") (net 3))
 (segment (start 127.632229 52.891943) (end 127.632229 83.323829) (width 0.25) (layer "F.Cu") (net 3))
 (segment (start 117.167429 88.734029) (end 117.167429 99.224229) (width 0.25) (layer "F.Cu") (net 3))
 (segment (start 156.105629 121.982629) (end 156.232629 121.855629) (width 0.25) (layer "F.Cu") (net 3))
 (segment (start 176.044629 121.601629) (end 176.425629 121.982629) (width 0.25) (layer "F.Cu") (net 3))
 (segment (start 119.301029 113.092629) (end 117.243629 111.035229) (width 0.25) (layer "F.Cu") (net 3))
 (segment (start 90.183571 67.550429) (end 95.044029 67.550429) (width 0.25) (layer "F.Cu") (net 3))
 (segment (start 133.931429 55.127141) (end 133.931429 110.197029) (width 0.25) (layer "F.Cu") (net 3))
 (segment (start 122.755429 83.146029) (end 117.167429 88.734029) (width 0.25) (layer "F.Cu") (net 3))
 (segment (start 85.892829 122.109629) (end 84.9122 121.129) (width 0.25) (layer "F.Cu") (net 3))
 (segment (start 156.232629 121.855629) (end 155.978629 122.109629) (width 0.25) (layer "F.Cu") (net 3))
 (segment (start 149.882629 121.982629) (end 149.374629 121.982629) (width 0.25) (layer "F.Cu") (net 3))
 (segment (start 162.963629 121.855629) (end 162.709629 122.109629) (width 0.25) (layer "F.Cu") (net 3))
 (segment (start 138.9126 47.326571) (end 137.600385 48.638785) (width 0.25) (layer "F.Cu") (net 3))
 (segment (start 140.4112 51.977458) (end 135.633229 56.755429) (width 0.25) (layer "F.Cu") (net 3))
 (segment (start 176.050151 121.665087) (end 176.066419 121.648819) (width 0.25) (layer "F.Cu") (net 3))
 (segment (start 119.783629 109.536629) (end 119.783629 104.278829) (width 0.25) (layer "F.Cu") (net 3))
 (segment (start 147.9296 51.085771) (end 141.3002 51.085771) (width 0.25) (layer "F.Cu") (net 3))
 (segment (start 176.171629 121.855629) (end 175.917629 122.109629) (width 0.25) (layer "F.Cu") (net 3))
 (segment (start 139.9032 49.155371) (end 139.645085 49.413485) (width 0.25) (layer "F.Cu") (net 3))
 (segment (start 137.600385 48.638785) (end 132.051829 54.187341) (width 0.25) (layer "F.Cu") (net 3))
 (segment (start 182.267629 121.982629) (end 182.648629 121.601629) (width 0.25) (layer "F.Cu") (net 3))
 (segment (start 169.694629 121.982629) (end 169.186629 121.982629) (width 0.25) (layer "F.Cu") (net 3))
 (segment (start 169.418 121.570771) (end 169.418 52.685971) (width 0.25) (layer "F.Cu") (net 3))
 (segment (start 143.758458 121.657887) (end 143.762746 121.653599) (width 0.25) (layer "F.Cu") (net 3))
 (segment (start 121.028229 104.264629) (end 122.284029 104.264629) (width 0.25) (layer "F.Cu") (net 3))
 (segment (start 162.8394 52.750804) (end 157.415167 47.326571) (width 0.25) (layer "F.Cu") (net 3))
 (segment (start 131.974285 42.453885) (end 122.755429 51.672741) (width 0.25) (layer "F.Cu") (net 3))
 (segment (start 169.059629 121.982629) (end 169.440629 121.601629) (width 0.25) (layer "F.Cu") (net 3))
 (segment (start 137.8204 45.573971) (end 136.762185 46.632185) (width 0.25) (layer "F.Cu") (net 3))
 (segment (start 169.313629 121.982629) (end 169.440629 121.855629) (width 0.25) (layer "F.Cu") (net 3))
 (segment (start 175.663629 121.982629) (end 176.044629 121.601629) (width 0.25) (layer "F.Cu") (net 3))
 (segment (start 117.243629 111.035229) (end 117.243629 104.278829) (width 0.25) (layer "F.Cu") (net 3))
 (segment (start 130.934229 110.527229) (end 120.774229 110.527229) (width 0.25) (layer "F.Cu") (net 3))
 (segment (start 129.816629 53.577741) (end 129.816629 83.704829) (width 0.25) (layer "F.Cu") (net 3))
 (segment (start 162.455629 121.982629) (end 162.836629 121.601629) (width 0.25) (layer "F.Cu") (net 3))
 (segment (start 120.774229 110.527229) (end 119.783629 109.536629) (width 0.25) (layer "F.Cu") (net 3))
 (segment (start 167.4622 43.999171) (end 136.525 43.999171) (width 0.25) (layer "F.Cu") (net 3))
 (segment (start 115.897429 111.568629) (end 115.897429 104.278829) (width 0.25) (layer "F.Cu") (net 3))
 (segment (start 85.6742 81.574) (end 85.6742 72.0598) (width 0.25) (layer "F.Cu") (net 3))
 (segment (start 169.418 52.685971) (end 162.306 45.573971) (width 0.25) (layer "F.Cu") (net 3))
 (segment (start 135.684029 110.781229) (end 133.372629 113.092629) (width 0.25) (layer "F.Cu") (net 3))
 (segment (start 139.645085 49.413485) (end 133.931429 55.127141) (width 0.25) (layer "F.Cu") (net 3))
 (segment (start 149.584888 52.741059) (end 147.9296 51.085771) (width 0.25) (layer "F.Cu") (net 3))
 (segment (start 128.597429 110.578029) (end 123.390429 105.371029) (width 0.25) (layer "B.Cu") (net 3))
 (segment (start 128.597429 121.500029) (end 128.597429 110.578029) (width 0.25) (layer "B.Cu") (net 3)))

